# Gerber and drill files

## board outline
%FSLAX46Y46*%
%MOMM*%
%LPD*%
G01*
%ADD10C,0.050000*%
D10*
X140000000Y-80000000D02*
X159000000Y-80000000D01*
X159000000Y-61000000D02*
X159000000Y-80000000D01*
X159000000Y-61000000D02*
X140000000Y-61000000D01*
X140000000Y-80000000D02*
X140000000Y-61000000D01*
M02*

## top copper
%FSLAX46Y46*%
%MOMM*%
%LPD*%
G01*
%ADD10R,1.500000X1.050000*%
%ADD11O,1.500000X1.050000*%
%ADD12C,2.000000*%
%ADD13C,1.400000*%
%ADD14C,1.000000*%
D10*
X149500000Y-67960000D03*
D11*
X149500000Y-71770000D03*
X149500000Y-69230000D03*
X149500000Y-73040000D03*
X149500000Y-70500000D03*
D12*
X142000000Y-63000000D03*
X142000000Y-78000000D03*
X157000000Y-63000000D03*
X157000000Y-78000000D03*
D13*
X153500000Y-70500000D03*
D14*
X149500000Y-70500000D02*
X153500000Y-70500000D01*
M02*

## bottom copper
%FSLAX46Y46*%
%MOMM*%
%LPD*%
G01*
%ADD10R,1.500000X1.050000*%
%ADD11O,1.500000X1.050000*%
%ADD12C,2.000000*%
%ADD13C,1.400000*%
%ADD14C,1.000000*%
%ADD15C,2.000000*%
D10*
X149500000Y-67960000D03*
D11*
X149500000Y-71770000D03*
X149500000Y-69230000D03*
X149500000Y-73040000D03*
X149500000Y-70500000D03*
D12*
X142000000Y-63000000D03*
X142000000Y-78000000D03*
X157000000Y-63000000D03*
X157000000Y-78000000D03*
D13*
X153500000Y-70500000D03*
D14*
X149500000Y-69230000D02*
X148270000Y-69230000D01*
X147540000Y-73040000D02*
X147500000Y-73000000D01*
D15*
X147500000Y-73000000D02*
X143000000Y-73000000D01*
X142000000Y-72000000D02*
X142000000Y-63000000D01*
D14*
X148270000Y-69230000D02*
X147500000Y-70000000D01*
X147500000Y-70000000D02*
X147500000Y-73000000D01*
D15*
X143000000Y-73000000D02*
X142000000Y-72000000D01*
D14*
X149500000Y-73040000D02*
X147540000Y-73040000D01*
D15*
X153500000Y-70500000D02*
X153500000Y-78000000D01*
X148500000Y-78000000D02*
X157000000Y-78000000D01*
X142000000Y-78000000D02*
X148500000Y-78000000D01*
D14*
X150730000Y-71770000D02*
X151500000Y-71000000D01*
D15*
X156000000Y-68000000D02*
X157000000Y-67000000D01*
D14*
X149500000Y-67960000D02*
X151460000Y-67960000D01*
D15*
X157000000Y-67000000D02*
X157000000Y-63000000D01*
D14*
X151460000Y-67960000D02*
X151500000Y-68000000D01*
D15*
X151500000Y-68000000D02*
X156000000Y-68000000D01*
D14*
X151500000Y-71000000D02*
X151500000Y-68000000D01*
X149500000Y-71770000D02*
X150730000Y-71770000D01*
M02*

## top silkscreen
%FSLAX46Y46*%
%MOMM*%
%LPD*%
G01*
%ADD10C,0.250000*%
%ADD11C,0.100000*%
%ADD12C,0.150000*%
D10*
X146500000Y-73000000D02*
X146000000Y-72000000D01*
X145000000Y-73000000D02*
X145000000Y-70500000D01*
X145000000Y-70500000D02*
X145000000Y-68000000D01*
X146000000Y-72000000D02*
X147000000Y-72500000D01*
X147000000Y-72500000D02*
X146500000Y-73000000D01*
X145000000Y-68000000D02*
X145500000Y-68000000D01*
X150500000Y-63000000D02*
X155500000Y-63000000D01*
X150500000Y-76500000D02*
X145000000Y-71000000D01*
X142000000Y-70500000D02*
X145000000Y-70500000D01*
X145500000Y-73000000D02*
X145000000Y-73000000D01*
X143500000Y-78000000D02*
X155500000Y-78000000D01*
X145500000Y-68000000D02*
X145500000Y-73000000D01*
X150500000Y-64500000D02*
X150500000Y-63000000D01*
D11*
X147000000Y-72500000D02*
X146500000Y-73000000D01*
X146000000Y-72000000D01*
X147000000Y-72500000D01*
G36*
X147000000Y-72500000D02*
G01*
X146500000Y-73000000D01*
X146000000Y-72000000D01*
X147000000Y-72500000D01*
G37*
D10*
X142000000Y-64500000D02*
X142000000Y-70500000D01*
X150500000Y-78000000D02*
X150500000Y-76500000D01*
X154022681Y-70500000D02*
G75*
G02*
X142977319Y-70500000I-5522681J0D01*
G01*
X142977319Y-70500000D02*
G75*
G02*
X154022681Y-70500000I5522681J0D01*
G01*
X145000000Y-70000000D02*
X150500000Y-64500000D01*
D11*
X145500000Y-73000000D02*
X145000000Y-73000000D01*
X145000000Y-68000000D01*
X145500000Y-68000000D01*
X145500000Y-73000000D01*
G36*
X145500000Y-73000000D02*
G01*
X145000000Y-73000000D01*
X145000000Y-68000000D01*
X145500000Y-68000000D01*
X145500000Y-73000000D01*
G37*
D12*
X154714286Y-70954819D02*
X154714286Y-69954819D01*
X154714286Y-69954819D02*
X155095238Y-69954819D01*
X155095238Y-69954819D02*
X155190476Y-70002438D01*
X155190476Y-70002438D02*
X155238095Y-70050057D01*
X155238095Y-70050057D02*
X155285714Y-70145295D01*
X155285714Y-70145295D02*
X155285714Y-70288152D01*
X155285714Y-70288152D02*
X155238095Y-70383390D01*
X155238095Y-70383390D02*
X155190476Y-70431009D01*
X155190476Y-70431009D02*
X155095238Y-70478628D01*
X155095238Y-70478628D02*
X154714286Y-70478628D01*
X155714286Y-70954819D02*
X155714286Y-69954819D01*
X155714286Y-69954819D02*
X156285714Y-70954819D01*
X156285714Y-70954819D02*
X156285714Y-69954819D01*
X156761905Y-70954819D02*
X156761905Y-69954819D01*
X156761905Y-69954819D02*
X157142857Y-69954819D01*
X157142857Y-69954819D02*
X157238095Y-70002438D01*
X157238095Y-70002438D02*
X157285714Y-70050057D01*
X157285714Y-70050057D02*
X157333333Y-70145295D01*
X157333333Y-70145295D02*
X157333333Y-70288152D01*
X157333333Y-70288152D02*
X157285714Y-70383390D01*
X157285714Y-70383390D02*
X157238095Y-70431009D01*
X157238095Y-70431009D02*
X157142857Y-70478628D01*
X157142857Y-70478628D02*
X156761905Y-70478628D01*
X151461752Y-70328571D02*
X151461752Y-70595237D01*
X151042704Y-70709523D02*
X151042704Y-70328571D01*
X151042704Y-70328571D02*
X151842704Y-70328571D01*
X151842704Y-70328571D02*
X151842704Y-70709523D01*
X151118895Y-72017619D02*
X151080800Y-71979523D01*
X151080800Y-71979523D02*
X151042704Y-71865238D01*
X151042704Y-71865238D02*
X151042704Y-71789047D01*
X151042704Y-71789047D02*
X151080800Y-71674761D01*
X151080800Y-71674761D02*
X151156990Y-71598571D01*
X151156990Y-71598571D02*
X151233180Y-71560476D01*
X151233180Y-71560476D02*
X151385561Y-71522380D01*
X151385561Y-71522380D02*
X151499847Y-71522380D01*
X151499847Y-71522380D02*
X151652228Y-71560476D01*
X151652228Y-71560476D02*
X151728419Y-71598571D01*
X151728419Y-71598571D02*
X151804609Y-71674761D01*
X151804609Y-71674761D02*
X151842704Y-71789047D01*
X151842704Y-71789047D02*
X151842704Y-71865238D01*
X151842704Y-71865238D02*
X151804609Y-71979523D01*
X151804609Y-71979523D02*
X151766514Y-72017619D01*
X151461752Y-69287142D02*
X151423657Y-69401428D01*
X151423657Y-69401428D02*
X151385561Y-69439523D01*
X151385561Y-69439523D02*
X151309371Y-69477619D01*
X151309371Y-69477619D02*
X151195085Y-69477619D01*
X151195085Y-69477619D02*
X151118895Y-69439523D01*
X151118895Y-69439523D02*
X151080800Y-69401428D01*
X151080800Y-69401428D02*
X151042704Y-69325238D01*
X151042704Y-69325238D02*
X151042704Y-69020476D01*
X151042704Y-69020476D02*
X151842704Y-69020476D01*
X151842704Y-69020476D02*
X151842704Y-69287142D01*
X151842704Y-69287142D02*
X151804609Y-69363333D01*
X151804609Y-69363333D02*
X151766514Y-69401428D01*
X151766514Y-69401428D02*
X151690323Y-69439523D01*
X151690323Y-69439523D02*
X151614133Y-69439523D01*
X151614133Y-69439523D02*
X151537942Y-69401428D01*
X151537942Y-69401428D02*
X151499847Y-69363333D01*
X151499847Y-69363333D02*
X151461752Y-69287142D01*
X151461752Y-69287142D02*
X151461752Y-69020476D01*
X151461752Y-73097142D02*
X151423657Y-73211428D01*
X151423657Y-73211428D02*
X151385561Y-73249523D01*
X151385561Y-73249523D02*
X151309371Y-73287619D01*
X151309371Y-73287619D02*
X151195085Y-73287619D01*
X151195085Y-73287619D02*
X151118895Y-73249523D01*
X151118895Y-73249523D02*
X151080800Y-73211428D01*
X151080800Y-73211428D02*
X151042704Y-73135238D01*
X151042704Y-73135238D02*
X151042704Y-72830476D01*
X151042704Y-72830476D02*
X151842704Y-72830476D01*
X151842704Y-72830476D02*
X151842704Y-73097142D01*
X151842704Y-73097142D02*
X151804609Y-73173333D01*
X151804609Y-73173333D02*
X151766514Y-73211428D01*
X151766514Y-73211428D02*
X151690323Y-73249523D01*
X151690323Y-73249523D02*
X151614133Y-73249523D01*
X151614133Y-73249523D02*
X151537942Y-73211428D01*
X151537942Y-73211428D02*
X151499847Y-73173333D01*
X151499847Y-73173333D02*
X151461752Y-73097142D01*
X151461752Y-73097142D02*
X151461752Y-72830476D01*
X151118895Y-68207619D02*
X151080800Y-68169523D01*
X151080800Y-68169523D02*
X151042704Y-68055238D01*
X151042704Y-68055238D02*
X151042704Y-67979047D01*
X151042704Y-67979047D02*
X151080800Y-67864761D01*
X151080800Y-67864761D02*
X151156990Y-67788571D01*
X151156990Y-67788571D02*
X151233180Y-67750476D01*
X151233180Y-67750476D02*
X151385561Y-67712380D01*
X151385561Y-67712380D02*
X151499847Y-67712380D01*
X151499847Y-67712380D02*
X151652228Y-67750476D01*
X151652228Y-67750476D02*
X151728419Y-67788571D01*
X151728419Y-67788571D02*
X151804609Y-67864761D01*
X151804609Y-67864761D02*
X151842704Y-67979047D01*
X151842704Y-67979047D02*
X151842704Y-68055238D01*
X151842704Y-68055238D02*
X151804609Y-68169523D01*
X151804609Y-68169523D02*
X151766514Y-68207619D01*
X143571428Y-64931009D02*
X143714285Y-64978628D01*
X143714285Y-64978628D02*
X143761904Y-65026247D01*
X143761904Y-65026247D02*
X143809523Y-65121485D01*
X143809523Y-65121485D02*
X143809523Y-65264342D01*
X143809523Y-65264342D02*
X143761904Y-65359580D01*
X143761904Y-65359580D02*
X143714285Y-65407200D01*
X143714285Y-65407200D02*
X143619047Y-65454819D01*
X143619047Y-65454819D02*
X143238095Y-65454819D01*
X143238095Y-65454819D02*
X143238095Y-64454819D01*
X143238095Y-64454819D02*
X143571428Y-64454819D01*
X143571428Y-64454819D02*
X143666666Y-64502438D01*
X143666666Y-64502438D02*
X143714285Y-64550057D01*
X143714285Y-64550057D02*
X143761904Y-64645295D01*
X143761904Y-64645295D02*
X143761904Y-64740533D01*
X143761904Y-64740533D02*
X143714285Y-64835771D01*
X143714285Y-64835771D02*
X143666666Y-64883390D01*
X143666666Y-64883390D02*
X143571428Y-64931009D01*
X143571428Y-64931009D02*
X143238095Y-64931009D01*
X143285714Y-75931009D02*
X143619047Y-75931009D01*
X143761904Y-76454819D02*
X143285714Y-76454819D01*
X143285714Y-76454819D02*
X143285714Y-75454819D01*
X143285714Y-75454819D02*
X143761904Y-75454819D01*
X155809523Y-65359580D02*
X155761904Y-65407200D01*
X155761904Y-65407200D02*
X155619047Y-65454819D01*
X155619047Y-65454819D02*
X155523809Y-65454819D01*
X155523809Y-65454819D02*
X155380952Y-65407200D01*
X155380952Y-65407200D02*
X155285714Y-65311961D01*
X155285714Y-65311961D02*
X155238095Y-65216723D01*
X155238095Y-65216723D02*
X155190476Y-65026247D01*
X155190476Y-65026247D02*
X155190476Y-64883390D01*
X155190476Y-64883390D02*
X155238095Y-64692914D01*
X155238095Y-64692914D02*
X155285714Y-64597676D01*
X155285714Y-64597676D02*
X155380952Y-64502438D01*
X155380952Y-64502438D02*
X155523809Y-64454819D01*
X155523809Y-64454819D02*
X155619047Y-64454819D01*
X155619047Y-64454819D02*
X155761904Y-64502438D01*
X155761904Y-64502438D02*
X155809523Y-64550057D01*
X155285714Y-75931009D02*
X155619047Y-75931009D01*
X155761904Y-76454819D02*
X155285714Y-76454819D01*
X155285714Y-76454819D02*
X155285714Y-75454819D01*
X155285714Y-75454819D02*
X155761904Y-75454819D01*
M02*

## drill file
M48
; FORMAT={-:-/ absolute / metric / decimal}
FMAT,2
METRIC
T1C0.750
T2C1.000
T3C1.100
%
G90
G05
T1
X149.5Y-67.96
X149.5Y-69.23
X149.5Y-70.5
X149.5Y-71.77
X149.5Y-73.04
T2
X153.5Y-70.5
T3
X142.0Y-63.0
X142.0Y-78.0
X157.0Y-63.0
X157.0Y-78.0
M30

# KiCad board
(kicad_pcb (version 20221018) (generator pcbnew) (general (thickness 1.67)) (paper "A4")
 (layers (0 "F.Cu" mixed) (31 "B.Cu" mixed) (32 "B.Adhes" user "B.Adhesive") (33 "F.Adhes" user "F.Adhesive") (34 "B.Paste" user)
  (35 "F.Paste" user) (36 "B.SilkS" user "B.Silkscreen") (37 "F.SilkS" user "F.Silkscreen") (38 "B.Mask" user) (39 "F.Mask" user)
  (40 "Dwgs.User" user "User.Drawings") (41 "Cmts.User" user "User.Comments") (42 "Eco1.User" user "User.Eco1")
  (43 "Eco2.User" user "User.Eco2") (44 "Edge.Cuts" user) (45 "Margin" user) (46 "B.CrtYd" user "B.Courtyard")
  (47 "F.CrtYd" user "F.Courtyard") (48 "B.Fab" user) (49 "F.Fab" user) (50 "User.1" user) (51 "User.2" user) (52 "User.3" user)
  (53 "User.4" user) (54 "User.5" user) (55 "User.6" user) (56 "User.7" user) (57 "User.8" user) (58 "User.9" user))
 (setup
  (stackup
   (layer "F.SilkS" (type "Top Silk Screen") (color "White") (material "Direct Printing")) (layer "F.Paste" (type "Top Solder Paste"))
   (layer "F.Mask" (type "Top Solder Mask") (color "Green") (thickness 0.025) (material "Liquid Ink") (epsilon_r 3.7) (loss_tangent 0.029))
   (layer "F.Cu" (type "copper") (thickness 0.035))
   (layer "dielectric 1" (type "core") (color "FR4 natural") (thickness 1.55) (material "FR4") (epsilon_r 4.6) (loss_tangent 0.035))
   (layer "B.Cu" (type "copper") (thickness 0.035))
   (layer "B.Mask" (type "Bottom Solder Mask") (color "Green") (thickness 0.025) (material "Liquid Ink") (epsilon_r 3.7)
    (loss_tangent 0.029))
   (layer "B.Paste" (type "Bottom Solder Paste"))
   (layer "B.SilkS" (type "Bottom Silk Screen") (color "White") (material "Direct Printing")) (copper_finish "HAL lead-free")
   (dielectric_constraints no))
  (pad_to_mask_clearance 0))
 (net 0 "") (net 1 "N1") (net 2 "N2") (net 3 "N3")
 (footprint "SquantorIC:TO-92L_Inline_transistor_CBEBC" (layer "F.Cu") (at 149.5 70.5 -90)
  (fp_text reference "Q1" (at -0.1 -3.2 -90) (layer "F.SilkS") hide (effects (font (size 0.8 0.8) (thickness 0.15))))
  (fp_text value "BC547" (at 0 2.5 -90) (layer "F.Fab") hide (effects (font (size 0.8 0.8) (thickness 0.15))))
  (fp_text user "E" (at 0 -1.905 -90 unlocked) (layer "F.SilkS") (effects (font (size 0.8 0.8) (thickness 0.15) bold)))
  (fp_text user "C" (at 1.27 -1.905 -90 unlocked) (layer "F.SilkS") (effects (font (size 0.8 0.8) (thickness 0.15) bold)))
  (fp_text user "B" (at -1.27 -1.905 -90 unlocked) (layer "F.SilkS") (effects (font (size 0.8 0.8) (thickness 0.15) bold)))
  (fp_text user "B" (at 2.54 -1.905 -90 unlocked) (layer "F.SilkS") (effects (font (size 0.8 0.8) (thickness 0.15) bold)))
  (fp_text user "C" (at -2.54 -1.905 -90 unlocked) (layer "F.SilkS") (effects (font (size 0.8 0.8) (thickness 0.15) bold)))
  (pad "1" thru_hole rect (at -2.54 0 270) (size 1.05 1.5) (drill 0.75) (layers "*.Cu" "*.Mask") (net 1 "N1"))
  (pad "1" thru_hole oval (at 1.27 0 270) (size 1.05 1.5) (drill 0.75) (layers "*.Cu" "*.Mask") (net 1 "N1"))
  (pad "2" thru_hole oval (at -1.27 0 270) (size 1.05 1.5) (drill 0.75) (layers "*.Cu" "*.Mask") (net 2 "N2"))
  (pad "2" thru_hole oval (at 2.54 0 270) (size 1.05 1.5) (drill 0.75) (layers "*.Cu" "*.Mask") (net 2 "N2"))
  (pad "3" thru_hole oval (at 0 0 270) (size 1.05 1.5) (drill 0.75) (layers "*.Cu" "*.Mask") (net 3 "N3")))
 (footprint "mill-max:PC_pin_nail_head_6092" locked (layer "F.Cu") (at 142 63)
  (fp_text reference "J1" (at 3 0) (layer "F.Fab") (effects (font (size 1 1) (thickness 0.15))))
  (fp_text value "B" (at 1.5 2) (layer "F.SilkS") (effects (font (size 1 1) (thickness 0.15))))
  (pad "1" thru_hole circle locked (at 0 0) (size 2 2) (drill 1.1) (layers "*.Cu" "*.Mask") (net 2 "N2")))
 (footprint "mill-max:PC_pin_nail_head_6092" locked (layer "F.Cu") (at 142 78)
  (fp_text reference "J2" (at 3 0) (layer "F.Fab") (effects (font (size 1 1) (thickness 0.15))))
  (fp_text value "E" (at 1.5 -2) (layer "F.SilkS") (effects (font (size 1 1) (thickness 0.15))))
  (pad "1" thru_hole circle locked (at 0 0) (size 2 2) (drill 1.1) (layers "*.Cu" "*.Mask") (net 3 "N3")))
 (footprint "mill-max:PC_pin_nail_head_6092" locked (layer "F.Cu") (at 157 63)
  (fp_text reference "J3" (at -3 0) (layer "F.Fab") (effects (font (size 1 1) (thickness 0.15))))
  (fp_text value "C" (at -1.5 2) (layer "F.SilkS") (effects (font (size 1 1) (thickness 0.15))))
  (pad "1" thru_hole circle locked (at 0 0) (size 2 2) (drill 1.1) (layers "*.Cu" "*.Mask") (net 1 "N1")))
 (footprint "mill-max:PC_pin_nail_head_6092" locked (layer "F.Cu") (at 157 78)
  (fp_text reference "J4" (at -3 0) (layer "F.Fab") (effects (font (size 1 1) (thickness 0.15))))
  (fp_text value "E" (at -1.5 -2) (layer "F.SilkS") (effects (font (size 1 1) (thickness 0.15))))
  (pad "1" thru_hole circle locked (at 0 0) (size 2 2) (drill 1.1) (layers "*.Cu" "*.Mask") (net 3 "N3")))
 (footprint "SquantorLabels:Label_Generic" (layer "B.Cu") (at 157.75 71.25 90)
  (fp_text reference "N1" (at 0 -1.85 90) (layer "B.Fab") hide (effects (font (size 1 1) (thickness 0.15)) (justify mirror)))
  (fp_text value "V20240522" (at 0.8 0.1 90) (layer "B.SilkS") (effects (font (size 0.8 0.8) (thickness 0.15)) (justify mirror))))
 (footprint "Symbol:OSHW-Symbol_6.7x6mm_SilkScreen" (layer "B.Cu") (at 154 70.5 -90)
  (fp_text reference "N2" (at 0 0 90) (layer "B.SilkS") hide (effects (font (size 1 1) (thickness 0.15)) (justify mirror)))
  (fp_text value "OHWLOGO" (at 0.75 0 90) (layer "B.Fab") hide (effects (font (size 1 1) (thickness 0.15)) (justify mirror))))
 (gr_line (start 146.5 73) (end 146 72) (stroke (width 0.25) (type solid)) (layer "F.SilkS"))
 (gr_line (start 145 73) (end 145 70.5) (stroke (width 0.25) (type solid)) (layer "F.SilkS"))
 (gr_line (start 145 70.5) (end 145 68) (stroke (width 0.25) (type solid)) (layer "F.SilkS"))
 (gr_line (start 146 72) (end 147 72.5) (stroke (width 0.25) (type solid)) (layer "F.SilkS"))
 (gr_line (start 147 72.5) (end 146.5 73) (stroke (width 0.25) (type solid)) (layer "F.SilkS"))
 (gr_line (start 145 68) (end 145.5 68) (stroke (width 0.25) (type solid)) (layer "F.SilkS"))
 (gr_line (start 150.5 63) (end 155.5 63) (stroke (width 0.25) (type solid)) (layer "F.SilkS"))
 (gr_line (start 150.5 76.5) (end 145 71) (stroke (width 0.25) (type solid)) (layer "F.SilkS"))
 (gr_line (start 142 70.5) (end 145 70.5) (stroke (width 0.25) (type solid)) (layer "F.SilkS"))
 (gr_line (start 145.5 73) (end 145 73) (stroke (width 0.25) (type solid)) (layer "F.SilkS"))
 (gr_line (start 143.5 78) (end 155.5 78) (stroke (width 0.25) (type solid)) (layer "F.SilkS"))
 (gr_line (start 145.5 68) (end 145.5 73) (stroke (width 0.25) (type solid)) (layer "F.SilkS"))
 (gr_line (start 150.5 64.5) (end 150.5 63) (stroke (width 0.25) (type solid)) (layer "F.SilkS"))
 (gr_poly (pts (xy 147 72.5) (xy 146.5 73) (xy 146 72)) (stroke (width 0.1) (type solid)) (fill solid) (layer "F.SilkS"))
 (gr_line (start 142 64.5) (end 142 70.5) (stroke (width 0.25) (type solid)) (layer "F.SilkS"))
 (gr_line (start 150.5 78) (end 150.5 76.5) (stroke (width 0.25) (type solid)) (layer "F.SilkS"))
 (gr_circle (center 148.5 70.5) (end 154 71) (stroke (width 0.25) (type solid)) (fill none) (layer "F.SilkS"))
 (gr_line (start 145 70) (end 150.5 64.5) (stroke (width 0.25) (type solid)) (layer "F.SilkS"))
 (gr_poly (pts (xy 145.5 73) (xy 145 73) (xy 145 68) (xy 145.5 68)) (stroke (width 0.1) (type solid)) (fill solid) (layer "F.SilkS"))
 (gr_line (start 140 80) (end 159 80) (stroke (width 0.05) (type solid)) (layer "Edge.Cuts"))
 (gr_line (start 159 61) (end 159 80) (stroke (width 0.05) (type solid)) (layer "Edge.Cuts"))
 (gr_line (start 159 61) (end 140 61) (stroke (width 0.05) (type solid)) (layer "Edge.Cuts"))
 (gr_line (start 140 80) (end 140 61) (stroke (width 0.05) (type solid)) (layer "Edge.Cuts"))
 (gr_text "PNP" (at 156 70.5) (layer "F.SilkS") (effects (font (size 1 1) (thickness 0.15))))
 (segment (start 149.5 69.23) (end 148.27 69.23) (width 1) (layer "B.Cu") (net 2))
 (segment (start 147.54 73.04) (end 147.5 73) (width 1) (layer "B.Cu") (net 2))
 (segment (start 147.5 73) (end 143 73) (width 2) (layer "B.Cu") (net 2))
 (segment (start 142 72) (end 142 63) (width 2) (layer "B.Cu") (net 2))
 (segment (start 148.27 69.23) (end 147.5 70) (width 1) (layer "B.Cu") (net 2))
 (segment (start 147.5 70) (end 147.5 73) (width 1) (layer "B.Cu") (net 2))
 (segment (start 143 73) (end 142 72) (width 2) (layer "B.Cu") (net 2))
 (segment (start 149.5 73.04) (end 147.54 73.04) (width 1) (layer "B.Cu") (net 2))
 (segment (start 149.5 70.5) (end 153.5 70.5) (width 1) (layer "F.Cu") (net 3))
 (via (at 153.5 70.5) (size 1.4) (drill 1) (layers "F.Cu" "B.Cu") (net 3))
 (segment (start 153.5 70.5) (end 153.5 78) (width 2) (layer "B.Cu") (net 3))
 (segment (start 148.5 78) (end 157 78) (width 2) (layer "B.Cu") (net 3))
 (segment (start 142 78) (end 148.5 78) (width 2) (layer "B.Cu") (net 3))
 (segment (start 150.73 71.77) (end 151.5 71) (width 1) (layer "B.Cu") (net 1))
 (segment (start 156 68) (end 157 67) (width 2) (layer "B.Cu") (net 1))
 (segment (start 149.5 67.96) (end 151.46 67.96) (width 1) (layer "B.Cu") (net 1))
 (segment (start 157 67) (end 157 63) (width 2) (layer "B.Cu") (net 1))
 (segment (start 151.46 67.96) (end 151.5 68) (width 1) (layer "B.Cu") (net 1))
 (segment (start 151.5 68) (end 156 68) (width 2) (layer "B.Cu") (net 1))
 (segment (start 151.5 71) (end 151.5 68) (width 1) (layer "B.Cu") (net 1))
 (segment (start 149.5 71.77) (end 150.73 71.77) (width 1) (layer "B.Cu") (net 1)))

